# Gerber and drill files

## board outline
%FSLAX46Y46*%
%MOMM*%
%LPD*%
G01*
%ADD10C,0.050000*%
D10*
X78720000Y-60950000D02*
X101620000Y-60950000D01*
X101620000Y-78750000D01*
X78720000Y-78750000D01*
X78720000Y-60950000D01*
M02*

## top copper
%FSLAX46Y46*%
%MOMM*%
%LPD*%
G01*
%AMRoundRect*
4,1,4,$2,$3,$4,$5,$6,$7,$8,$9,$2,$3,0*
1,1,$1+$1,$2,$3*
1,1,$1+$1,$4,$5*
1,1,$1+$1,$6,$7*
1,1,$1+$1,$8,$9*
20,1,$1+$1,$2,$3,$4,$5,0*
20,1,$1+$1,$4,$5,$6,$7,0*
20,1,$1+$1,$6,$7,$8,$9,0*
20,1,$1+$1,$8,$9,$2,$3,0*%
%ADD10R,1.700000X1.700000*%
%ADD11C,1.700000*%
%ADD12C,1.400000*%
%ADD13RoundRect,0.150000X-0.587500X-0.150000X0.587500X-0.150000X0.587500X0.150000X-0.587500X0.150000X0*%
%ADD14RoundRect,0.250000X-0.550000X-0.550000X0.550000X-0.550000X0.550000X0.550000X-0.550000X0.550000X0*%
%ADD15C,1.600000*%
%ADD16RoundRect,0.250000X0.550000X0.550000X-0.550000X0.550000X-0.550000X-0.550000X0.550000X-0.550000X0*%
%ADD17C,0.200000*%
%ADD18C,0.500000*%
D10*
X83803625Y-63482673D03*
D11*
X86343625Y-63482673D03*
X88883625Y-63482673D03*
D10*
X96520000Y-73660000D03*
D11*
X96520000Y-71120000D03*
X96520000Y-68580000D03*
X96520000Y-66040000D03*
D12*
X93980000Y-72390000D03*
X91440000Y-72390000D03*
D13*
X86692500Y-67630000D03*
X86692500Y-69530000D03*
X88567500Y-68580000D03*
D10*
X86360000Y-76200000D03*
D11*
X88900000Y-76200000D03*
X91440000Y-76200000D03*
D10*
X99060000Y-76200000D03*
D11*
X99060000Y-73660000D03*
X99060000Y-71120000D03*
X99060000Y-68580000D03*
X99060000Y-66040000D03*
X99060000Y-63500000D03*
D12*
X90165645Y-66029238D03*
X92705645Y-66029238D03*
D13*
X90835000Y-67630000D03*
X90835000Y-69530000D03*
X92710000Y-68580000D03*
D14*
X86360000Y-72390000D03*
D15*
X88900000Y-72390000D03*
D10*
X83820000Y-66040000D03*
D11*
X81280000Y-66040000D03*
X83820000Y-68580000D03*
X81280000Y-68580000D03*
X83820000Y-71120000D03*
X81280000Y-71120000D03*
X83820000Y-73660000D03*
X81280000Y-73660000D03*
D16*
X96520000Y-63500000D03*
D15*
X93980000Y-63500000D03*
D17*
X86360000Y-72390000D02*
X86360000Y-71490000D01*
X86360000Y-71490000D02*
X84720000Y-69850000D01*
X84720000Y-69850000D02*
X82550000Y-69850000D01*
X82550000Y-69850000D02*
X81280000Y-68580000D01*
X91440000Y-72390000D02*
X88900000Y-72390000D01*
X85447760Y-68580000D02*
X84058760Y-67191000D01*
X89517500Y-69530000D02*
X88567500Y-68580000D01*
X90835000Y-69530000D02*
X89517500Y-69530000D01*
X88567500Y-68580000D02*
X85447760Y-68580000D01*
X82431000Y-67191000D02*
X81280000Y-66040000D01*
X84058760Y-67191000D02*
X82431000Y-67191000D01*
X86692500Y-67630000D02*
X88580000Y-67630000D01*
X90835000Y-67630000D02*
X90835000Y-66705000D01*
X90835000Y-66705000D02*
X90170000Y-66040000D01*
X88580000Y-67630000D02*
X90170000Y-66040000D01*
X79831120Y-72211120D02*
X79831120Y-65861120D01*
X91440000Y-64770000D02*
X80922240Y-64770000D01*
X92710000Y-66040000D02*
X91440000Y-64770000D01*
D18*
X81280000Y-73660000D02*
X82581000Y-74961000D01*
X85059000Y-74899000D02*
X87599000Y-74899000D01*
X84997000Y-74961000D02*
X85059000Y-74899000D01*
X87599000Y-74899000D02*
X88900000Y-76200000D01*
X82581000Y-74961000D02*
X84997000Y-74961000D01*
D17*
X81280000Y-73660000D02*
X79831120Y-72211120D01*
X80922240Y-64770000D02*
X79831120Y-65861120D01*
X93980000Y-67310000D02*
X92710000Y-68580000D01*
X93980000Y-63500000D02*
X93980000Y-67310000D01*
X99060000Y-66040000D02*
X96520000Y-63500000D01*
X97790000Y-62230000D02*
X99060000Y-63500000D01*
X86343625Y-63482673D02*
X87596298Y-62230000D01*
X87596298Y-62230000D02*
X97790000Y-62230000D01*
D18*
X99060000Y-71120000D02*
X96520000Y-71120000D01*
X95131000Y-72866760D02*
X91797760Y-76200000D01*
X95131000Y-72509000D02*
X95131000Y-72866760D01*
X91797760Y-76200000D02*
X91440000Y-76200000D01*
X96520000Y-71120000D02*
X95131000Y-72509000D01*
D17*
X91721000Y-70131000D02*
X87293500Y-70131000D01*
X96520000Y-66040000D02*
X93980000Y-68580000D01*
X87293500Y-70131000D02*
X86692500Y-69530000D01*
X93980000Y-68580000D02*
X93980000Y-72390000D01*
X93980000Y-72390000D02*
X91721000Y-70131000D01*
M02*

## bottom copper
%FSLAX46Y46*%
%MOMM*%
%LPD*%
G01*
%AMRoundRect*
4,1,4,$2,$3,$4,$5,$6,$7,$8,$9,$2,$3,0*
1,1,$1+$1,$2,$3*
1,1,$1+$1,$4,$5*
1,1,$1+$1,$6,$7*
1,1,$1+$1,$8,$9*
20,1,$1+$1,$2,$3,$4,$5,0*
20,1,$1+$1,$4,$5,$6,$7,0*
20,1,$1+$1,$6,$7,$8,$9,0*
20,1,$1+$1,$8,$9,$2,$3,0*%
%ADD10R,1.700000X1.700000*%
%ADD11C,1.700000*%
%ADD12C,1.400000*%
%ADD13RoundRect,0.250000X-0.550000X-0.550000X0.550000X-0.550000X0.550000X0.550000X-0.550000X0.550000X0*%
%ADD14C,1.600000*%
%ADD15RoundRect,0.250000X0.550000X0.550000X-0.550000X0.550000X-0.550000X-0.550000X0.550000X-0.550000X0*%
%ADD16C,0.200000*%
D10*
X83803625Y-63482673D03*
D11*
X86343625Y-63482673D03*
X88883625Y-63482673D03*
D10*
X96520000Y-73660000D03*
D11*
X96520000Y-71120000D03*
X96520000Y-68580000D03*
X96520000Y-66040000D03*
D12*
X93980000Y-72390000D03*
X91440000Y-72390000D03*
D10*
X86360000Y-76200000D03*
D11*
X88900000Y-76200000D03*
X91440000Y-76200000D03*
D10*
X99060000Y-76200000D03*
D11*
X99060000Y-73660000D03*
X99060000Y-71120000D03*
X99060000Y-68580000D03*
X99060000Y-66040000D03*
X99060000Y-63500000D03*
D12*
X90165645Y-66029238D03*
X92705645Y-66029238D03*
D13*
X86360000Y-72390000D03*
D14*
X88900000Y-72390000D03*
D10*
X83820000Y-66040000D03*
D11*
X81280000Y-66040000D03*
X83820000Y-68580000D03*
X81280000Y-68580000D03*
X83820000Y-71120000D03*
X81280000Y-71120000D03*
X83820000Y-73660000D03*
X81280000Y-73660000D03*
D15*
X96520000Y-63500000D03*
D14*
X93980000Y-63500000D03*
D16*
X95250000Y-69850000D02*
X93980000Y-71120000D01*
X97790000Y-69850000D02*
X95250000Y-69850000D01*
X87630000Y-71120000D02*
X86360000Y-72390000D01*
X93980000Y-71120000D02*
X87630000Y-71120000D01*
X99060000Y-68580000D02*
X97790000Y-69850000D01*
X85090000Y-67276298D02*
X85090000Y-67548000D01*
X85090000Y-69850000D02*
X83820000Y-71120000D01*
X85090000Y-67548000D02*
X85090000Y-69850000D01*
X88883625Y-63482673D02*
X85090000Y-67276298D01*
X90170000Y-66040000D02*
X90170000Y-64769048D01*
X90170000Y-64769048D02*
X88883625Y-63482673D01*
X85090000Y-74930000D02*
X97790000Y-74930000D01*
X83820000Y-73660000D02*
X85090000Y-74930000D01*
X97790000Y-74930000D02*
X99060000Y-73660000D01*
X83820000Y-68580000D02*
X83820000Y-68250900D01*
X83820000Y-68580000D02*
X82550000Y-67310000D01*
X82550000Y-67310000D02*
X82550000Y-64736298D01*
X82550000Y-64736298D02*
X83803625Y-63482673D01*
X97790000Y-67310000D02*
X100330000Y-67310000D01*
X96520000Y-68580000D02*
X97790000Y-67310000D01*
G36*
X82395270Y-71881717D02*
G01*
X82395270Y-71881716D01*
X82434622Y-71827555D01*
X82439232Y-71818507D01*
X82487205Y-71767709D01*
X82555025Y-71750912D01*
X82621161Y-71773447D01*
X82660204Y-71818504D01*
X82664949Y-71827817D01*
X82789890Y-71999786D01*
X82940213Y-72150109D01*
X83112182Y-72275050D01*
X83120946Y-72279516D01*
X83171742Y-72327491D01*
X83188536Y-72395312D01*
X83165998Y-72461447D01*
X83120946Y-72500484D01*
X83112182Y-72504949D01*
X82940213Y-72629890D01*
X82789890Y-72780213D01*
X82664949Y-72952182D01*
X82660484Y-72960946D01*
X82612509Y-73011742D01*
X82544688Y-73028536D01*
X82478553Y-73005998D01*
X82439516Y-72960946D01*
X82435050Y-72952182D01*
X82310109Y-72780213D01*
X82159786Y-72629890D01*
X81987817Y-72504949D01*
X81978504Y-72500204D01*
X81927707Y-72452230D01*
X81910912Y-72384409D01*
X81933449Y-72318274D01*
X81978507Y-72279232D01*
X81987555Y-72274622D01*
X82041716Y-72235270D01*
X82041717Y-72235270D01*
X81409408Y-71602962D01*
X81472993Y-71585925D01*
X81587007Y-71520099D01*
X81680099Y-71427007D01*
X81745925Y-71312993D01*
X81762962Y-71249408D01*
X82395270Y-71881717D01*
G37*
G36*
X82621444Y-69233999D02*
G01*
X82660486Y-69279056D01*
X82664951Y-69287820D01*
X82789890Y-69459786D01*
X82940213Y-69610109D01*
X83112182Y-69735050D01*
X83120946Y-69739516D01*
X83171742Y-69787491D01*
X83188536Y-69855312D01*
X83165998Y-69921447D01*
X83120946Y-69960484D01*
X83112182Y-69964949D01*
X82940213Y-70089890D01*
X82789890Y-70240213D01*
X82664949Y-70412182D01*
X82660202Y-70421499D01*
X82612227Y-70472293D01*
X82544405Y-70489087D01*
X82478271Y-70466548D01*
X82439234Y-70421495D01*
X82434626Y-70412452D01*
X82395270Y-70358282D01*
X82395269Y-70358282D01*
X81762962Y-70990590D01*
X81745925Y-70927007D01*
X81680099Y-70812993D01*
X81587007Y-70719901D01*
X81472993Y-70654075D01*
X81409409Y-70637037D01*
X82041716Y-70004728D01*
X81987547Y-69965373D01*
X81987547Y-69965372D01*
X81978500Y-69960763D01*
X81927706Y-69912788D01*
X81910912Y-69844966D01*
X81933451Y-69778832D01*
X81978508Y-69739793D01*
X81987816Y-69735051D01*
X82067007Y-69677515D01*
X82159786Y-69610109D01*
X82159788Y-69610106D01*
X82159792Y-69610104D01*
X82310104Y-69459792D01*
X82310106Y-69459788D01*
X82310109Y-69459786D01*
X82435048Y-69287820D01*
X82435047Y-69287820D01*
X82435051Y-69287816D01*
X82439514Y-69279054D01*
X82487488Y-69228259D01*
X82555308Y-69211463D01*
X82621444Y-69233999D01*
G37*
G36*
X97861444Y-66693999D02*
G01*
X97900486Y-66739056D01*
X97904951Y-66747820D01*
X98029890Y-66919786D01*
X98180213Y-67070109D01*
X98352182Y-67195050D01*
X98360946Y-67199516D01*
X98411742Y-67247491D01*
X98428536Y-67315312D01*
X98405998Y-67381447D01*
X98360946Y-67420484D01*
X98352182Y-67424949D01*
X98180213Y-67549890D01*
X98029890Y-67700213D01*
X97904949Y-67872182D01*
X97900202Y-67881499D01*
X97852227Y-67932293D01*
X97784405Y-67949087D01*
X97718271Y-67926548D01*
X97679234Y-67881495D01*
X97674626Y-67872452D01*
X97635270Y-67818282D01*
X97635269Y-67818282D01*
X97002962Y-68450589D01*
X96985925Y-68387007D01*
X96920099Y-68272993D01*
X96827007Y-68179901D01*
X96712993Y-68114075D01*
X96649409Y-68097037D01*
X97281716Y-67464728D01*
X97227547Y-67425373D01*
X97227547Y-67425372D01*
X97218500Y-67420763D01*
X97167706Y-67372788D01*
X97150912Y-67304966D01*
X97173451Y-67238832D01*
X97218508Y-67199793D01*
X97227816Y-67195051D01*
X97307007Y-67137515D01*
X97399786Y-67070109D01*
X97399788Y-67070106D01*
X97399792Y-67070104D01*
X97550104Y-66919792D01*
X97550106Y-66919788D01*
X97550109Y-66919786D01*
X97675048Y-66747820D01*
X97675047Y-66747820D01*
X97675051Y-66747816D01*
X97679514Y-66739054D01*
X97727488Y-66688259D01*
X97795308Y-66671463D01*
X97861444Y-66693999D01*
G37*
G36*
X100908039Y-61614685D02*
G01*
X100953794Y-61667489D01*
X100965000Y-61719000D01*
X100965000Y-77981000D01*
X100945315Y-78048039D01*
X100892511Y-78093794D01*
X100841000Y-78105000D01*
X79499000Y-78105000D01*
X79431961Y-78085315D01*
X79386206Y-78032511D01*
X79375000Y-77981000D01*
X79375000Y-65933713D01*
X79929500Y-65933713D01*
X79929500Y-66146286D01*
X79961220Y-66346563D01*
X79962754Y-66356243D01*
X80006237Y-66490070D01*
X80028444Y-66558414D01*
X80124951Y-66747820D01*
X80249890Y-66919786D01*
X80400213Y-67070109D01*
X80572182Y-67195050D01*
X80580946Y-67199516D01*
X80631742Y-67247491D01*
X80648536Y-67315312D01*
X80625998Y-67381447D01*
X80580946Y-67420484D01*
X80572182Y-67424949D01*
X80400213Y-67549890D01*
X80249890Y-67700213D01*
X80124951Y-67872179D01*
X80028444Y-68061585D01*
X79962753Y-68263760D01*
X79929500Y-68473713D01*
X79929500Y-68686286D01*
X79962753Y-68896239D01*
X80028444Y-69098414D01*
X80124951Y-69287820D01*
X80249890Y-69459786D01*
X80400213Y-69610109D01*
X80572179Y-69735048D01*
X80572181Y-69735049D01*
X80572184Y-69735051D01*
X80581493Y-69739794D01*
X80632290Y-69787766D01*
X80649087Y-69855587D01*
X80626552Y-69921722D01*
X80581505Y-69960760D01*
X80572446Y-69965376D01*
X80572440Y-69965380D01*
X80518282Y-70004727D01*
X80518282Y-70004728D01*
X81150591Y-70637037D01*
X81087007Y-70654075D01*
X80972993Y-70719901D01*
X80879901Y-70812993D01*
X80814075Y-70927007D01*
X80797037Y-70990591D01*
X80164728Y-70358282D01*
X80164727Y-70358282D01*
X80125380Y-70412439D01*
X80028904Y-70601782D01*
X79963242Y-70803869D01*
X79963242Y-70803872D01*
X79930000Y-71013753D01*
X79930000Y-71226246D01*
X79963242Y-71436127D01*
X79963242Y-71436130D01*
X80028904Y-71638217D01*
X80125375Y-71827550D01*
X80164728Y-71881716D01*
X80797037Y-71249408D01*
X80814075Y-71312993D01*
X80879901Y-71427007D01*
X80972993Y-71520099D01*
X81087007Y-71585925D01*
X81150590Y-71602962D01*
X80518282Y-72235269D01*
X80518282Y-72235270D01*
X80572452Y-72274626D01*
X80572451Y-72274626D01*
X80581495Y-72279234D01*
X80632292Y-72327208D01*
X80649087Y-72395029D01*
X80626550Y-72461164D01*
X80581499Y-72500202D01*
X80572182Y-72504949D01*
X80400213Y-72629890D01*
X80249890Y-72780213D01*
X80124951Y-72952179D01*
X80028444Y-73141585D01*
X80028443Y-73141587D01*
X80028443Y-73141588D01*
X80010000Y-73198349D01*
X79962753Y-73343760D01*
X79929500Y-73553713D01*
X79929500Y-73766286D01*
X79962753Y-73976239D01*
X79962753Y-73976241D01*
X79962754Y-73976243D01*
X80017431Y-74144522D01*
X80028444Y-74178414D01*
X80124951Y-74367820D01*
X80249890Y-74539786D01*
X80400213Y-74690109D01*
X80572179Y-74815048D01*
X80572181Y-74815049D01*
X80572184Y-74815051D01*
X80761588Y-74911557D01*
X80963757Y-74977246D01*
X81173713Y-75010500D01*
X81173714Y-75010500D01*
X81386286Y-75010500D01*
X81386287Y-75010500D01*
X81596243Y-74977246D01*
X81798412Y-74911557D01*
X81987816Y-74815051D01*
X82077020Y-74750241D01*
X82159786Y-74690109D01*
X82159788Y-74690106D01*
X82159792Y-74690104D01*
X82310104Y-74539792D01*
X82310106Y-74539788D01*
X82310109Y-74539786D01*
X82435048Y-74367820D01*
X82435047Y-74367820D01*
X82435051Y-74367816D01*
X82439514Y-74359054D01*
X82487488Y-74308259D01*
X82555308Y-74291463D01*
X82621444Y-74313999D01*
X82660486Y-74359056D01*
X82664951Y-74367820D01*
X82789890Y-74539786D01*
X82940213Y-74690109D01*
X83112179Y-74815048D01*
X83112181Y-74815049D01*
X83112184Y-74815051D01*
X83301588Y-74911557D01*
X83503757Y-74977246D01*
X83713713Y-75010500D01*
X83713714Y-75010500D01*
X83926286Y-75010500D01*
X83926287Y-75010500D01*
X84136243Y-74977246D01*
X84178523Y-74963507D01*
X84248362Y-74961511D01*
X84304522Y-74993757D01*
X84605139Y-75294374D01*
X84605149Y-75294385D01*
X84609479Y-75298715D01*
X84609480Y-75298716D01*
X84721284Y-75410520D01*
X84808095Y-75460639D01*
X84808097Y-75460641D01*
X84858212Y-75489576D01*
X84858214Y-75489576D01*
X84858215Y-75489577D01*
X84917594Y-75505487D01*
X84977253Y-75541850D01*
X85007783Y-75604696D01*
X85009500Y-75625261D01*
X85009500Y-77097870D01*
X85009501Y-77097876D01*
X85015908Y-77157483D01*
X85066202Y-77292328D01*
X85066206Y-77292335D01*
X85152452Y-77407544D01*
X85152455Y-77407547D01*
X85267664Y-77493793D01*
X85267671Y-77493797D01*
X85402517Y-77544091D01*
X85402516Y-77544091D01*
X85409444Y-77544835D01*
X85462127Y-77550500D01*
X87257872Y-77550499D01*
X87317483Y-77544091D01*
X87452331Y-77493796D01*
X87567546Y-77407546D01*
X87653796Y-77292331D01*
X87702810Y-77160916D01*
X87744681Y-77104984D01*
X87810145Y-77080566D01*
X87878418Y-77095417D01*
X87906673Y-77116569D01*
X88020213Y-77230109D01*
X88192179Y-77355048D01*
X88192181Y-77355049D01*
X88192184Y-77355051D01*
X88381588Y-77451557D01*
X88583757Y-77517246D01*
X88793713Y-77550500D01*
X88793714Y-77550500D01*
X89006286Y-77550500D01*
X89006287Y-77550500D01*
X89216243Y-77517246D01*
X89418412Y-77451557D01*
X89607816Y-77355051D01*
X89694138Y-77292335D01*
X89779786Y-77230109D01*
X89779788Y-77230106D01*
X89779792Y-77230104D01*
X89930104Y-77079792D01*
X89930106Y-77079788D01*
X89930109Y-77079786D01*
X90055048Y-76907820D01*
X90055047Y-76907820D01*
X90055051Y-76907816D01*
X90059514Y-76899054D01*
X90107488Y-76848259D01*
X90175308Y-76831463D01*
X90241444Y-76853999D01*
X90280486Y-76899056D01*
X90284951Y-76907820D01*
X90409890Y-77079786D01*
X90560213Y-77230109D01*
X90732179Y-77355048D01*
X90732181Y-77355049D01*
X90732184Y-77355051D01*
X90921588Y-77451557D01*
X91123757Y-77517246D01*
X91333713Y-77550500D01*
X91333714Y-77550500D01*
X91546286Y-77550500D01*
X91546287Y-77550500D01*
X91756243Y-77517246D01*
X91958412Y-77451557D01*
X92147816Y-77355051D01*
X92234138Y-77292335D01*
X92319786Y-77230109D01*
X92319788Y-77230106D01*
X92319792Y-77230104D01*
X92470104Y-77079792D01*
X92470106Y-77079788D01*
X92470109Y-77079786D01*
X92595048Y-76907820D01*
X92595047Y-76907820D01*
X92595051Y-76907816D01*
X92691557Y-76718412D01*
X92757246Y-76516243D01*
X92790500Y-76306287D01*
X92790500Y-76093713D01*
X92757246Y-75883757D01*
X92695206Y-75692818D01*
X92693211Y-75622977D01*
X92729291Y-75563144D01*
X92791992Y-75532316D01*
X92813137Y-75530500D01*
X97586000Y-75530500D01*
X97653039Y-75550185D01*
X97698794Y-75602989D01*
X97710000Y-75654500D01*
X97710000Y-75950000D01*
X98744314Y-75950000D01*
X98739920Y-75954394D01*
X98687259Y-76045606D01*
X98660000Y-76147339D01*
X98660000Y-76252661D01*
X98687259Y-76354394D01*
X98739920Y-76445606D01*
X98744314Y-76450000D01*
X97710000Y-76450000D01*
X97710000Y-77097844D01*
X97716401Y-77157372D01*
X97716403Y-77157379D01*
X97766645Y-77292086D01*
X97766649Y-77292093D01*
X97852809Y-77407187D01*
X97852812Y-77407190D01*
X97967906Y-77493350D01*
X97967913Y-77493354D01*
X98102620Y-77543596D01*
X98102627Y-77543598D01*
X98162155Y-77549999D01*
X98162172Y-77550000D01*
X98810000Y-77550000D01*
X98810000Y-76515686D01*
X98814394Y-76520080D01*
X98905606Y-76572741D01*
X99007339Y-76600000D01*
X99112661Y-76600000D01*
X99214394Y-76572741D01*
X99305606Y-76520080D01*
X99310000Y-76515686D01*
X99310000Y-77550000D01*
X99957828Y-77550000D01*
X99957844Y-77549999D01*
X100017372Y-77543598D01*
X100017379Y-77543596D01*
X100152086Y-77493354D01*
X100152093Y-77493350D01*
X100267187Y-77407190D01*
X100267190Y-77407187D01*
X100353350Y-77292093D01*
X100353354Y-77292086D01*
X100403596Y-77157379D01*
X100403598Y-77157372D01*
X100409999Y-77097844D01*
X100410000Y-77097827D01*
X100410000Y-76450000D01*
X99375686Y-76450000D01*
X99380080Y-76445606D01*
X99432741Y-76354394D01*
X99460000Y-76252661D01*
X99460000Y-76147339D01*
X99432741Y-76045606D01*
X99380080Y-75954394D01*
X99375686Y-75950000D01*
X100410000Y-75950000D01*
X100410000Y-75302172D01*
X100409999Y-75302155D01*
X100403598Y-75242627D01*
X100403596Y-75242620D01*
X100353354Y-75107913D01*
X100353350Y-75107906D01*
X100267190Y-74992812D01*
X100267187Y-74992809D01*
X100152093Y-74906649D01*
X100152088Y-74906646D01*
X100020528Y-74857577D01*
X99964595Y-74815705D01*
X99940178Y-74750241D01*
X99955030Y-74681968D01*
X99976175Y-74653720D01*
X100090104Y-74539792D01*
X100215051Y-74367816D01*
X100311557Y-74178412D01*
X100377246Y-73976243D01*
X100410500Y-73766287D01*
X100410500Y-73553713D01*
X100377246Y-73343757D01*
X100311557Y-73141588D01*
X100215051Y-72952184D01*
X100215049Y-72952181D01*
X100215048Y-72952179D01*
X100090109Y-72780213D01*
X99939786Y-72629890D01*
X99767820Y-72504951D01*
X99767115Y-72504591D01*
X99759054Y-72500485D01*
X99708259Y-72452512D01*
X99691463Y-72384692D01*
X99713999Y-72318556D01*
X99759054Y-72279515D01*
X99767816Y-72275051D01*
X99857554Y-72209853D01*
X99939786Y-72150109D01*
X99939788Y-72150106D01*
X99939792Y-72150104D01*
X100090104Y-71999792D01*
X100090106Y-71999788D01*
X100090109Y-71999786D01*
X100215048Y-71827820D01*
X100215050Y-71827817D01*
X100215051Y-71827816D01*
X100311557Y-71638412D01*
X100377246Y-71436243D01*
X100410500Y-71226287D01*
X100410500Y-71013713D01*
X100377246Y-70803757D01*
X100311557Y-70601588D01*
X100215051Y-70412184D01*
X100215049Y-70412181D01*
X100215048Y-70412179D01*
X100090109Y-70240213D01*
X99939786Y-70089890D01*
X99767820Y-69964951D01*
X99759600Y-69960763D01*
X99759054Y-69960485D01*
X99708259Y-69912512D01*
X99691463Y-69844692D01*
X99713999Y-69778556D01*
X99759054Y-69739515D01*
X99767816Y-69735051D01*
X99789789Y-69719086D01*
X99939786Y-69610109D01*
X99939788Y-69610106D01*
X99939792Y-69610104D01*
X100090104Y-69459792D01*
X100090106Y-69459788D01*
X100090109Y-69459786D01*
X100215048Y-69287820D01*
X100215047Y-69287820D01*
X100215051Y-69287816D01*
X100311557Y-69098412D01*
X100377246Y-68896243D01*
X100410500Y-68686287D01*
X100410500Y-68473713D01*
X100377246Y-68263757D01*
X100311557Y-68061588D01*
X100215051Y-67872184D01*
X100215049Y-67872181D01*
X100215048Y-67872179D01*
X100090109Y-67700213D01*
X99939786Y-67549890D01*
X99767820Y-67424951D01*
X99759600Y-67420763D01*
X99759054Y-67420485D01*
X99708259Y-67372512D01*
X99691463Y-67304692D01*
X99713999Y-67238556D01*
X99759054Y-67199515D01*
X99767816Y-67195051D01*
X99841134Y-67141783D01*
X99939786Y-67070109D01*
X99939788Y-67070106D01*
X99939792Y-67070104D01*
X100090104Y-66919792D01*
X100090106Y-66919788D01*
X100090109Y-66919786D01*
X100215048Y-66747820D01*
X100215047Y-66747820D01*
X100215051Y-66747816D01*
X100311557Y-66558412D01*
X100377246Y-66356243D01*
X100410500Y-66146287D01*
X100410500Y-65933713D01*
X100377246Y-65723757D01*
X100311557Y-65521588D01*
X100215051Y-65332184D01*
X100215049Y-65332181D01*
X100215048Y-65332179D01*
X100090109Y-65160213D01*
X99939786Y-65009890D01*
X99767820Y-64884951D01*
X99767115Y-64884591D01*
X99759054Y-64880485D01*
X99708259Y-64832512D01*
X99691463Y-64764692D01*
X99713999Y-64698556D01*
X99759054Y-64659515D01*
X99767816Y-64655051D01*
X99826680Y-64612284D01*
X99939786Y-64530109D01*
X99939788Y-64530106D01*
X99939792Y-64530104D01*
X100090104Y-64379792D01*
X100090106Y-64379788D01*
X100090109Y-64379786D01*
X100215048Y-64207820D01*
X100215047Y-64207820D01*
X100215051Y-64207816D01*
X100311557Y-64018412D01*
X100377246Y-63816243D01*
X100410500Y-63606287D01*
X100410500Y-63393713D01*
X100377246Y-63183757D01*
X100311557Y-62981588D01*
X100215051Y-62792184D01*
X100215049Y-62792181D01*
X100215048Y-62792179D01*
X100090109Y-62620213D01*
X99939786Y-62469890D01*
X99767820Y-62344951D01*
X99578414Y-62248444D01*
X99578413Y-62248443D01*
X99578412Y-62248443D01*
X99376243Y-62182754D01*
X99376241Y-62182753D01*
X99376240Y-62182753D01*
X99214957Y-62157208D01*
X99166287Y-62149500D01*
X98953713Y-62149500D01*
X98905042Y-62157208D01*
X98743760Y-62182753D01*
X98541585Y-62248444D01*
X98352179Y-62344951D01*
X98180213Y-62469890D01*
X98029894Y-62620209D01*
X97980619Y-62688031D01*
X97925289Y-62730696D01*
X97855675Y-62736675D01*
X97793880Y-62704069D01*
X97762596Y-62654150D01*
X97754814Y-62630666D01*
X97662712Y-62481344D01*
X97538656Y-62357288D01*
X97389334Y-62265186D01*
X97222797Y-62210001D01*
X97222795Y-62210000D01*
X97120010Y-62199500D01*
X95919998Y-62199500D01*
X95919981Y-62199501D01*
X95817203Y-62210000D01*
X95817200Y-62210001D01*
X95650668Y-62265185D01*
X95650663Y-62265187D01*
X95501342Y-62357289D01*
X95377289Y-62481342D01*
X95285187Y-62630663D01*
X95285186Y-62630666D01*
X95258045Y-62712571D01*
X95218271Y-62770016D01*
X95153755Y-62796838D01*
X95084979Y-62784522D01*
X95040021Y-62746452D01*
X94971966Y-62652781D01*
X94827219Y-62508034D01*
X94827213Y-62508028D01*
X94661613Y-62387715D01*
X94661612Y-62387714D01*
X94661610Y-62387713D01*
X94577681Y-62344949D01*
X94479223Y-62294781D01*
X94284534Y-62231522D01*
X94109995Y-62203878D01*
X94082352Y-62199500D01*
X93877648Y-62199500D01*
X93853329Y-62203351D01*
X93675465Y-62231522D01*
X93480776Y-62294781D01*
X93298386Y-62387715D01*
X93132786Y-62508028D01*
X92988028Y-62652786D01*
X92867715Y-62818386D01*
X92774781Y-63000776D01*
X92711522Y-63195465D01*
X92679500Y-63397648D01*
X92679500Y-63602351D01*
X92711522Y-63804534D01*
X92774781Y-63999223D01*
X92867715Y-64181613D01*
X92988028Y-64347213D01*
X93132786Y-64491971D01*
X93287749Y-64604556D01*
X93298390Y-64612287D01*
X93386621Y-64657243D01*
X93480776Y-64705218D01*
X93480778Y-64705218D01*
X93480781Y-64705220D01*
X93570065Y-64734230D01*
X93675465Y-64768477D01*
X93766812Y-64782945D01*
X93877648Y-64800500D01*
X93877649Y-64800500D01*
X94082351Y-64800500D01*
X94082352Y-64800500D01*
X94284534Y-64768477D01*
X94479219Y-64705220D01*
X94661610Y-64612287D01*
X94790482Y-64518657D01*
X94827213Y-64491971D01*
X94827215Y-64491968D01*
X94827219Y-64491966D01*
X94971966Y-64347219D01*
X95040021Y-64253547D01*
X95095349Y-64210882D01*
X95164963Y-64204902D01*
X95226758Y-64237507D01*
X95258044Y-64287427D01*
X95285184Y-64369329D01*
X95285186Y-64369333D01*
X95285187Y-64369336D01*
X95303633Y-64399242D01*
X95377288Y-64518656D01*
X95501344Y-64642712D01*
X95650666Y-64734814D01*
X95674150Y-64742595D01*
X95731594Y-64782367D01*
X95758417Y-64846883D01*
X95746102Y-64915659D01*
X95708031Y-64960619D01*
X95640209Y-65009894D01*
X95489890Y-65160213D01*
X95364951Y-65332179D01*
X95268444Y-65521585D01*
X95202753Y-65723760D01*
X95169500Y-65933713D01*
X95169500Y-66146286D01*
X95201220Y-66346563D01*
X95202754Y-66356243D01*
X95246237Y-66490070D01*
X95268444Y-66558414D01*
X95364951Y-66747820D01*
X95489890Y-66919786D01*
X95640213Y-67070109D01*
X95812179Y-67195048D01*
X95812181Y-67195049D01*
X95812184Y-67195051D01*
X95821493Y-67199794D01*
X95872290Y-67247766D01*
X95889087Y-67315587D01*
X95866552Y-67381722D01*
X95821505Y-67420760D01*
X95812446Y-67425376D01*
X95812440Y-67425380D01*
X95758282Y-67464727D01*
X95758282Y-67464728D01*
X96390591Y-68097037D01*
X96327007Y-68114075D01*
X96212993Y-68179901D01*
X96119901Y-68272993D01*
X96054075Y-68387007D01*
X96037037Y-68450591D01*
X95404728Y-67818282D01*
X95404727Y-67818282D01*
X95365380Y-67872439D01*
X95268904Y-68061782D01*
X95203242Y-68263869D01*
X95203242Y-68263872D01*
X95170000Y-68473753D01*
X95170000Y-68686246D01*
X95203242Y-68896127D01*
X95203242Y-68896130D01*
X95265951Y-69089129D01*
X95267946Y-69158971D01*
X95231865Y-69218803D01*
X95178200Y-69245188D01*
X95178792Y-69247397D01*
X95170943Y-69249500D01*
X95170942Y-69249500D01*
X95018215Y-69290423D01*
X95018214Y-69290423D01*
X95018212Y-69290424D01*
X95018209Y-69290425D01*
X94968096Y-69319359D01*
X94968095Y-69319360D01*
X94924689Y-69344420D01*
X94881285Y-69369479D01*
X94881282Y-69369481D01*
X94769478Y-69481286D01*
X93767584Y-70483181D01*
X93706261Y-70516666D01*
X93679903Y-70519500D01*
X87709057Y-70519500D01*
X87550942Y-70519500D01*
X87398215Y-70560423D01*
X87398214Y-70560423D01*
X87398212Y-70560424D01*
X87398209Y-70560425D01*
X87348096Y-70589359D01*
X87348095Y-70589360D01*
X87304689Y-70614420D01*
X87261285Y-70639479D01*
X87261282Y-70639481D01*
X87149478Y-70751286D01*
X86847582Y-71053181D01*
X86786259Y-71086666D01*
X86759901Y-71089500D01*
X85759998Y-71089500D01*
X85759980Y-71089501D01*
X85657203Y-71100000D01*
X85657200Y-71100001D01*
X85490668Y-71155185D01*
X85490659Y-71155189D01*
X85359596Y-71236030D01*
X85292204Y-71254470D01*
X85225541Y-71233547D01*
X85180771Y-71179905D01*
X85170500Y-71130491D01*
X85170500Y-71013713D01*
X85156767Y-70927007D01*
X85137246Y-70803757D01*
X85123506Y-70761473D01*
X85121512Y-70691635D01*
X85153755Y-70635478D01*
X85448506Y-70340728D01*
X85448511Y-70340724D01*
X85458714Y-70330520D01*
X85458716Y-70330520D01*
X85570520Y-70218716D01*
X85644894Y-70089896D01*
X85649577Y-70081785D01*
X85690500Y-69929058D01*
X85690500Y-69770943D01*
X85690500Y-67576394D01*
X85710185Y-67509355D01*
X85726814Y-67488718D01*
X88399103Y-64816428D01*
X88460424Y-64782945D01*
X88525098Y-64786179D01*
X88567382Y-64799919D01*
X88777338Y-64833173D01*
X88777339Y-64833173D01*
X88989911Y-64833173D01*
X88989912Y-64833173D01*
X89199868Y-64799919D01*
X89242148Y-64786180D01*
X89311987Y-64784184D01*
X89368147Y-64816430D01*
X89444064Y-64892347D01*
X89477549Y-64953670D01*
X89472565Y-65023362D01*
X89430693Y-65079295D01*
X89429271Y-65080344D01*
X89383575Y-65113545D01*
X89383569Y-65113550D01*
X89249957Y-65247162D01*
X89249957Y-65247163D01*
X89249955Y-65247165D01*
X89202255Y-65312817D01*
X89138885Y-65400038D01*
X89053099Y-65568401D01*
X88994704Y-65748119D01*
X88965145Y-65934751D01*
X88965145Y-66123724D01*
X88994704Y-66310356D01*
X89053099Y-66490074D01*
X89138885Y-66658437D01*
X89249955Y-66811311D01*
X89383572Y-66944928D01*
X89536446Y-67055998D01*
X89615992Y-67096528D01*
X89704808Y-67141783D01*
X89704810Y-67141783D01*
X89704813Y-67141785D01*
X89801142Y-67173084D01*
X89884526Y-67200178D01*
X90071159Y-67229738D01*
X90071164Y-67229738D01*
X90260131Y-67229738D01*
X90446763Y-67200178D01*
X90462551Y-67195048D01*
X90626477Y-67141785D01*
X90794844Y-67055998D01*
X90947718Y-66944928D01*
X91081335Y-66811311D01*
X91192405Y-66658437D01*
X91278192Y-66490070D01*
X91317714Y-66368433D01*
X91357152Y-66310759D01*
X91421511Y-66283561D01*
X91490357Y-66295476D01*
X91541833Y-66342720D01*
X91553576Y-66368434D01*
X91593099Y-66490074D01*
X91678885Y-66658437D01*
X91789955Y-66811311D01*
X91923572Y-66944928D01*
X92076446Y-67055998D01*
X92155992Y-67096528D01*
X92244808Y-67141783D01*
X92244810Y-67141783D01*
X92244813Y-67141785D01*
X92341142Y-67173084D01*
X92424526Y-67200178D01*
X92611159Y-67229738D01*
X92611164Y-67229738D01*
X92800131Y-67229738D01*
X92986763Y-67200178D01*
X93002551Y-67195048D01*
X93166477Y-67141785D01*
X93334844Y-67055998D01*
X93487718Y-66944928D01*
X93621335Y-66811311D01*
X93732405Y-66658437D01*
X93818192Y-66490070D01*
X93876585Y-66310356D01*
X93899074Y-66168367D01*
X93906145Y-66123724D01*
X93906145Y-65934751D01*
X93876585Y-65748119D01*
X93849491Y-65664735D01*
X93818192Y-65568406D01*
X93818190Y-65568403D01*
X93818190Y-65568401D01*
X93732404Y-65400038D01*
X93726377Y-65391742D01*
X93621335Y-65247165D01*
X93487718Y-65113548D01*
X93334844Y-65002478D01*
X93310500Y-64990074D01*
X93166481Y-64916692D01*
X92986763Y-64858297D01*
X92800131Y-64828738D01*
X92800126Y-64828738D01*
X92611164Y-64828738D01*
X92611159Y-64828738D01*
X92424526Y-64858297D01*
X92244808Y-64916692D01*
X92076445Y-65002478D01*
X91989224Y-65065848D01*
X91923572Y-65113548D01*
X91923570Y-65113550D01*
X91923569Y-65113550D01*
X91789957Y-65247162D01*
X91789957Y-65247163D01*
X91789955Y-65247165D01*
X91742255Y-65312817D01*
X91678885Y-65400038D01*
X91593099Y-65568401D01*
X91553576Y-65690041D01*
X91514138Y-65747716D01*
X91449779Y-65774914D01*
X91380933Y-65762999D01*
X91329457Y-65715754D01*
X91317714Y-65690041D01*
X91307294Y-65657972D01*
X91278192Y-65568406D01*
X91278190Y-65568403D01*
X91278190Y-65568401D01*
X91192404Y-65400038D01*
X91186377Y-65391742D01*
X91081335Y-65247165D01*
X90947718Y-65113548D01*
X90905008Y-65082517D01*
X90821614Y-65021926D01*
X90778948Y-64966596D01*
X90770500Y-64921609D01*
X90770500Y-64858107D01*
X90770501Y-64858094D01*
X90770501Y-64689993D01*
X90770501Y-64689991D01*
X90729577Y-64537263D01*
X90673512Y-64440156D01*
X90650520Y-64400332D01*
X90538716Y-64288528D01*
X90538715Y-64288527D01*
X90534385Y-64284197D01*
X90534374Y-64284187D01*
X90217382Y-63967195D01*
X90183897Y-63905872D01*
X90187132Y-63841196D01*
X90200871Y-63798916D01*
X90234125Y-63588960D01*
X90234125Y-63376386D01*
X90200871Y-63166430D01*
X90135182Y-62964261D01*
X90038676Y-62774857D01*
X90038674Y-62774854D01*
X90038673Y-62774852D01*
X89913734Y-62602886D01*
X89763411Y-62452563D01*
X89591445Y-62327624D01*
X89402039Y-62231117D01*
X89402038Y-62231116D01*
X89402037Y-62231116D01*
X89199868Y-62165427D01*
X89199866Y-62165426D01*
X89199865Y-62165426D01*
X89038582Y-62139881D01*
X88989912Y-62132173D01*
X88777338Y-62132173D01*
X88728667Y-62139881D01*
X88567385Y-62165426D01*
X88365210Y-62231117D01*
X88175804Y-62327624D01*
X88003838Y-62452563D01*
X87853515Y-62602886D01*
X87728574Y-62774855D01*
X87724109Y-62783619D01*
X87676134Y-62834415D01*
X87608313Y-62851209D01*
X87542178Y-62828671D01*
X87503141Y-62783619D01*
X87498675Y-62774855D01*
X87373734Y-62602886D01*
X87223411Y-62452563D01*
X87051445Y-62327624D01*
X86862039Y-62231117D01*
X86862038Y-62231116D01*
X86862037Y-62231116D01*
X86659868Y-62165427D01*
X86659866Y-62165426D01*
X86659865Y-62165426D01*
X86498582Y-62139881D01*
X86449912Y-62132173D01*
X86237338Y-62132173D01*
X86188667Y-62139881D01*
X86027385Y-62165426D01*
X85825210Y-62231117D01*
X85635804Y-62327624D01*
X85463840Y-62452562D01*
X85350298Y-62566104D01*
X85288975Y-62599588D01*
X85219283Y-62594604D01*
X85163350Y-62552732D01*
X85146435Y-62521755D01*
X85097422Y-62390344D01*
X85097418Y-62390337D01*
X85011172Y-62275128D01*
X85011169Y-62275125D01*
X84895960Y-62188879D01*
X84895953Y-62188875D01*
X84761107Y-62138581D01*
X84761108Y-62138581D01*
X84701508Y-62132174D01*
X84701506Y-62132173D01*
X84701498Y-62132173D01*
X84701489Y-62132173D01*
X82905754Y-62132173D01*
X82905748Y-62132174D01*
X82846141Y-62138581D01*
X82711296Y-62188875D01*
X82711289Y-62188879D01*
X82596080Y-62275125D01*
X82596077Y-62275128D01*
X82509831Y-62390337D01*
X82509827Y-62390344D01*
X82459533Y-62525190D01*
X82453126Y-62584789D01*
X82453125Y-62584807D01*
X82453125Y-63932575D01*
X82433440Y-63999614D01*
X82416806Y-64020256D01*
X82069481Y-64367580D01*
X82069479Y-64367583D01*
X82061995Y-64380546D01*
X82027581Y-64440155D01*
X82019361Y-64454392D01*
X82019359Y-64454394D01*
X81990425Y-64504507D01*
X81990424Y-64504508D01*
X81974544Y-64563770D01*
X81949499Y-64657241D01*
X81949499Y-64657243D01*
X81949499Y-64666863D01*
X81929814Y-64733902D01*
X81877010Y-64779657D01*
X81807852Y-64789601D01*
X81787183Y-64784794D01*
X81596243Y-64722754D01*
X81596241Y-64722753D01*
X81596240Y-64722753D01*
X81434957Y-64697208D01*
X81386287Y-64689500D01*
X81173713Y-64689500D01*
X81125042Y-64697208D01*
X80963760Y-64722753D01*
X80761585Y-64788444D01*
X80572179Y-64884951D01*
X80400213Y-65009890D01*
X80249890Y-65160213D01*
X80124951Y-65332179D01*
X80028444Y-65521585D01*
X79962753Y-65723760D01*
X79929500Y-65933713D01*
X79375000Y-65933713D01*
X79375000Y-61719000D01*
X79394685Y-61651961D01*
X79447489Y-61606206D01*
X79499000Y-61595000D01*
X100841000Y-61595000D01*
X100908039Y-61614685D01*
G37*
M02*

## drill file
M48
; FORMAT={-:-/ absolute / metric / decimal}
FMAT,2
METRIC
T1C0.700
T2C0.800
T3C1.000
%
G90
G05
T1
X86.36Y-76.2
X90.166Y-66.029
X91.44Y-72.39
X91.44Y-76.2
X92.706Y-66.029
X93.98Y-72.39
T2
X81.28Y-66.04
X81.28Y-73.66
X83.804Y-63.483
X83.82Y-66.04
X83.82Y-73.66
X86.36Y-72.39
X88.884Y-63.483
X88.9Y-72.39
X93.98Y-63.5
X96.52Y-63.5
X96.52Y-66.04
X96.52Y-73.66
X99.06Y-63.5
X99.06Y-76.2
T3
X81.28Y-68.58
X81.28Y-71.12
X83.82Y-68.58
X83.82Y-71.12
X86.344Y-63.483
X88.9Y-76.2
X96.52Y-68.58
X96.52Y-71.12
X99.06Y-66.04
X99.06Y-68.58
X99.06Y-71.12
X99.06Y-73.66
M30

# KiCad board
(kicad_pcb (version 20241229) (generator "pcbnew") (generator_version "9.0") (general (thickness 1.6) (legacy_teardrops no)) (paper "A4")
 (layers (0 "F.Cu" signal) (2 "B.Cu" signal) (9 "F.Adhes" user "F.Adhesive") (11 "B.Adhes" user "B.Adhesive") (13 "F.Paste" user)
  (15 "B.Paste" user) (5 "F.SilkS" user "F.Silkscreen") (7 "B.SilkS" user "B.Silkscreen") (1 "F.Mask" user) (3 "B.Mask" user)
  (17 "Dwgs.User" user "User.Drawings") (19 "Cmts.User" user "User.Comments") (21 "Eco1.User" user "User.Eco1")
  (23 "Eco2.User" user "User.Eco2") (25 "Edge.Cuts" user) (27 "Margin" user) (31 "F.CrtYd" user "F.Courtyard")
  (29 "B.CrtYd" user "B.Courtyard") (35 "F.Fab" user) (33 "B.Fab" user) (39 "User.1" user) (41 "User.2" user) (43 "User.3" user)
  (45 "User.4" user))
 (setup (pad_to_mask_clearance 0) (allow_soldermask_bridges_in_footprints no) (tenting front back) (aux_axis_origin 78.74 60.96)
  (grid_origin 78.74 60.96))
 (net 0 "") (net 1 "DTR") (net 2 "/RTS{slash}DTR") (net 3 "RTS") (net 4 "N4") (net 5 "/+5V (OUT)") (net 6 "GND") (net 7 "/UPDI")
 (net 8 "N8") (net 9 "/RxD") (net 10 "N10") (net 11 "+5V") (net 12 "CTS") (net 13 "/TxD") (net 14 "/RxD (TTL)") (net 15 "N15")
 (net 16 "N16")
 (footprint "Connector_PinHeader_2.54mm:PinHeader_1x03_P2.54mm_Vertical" (layer "F.Cu") (at 83.803625 63.482673 90)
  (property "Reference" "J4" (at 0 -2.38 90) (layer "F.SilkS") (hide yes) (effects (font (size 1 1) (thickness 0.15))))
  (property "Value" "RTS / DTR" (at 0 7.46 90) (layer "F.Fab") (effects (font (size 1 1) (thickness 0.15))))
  (pad "1" thru_hole rect (at 0 0 90) (size 1.7 1.7) (drill 0.8) (layers "*.Cu" "*.Mask") (remove_unused_layers no) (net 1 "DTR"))
  (pad "2" thru_hole circle (at 0 2.54 90) (size 1.7 1.7) (drill 1) (layers "*.Cu" "*.Mask") (remove_unused_layers no)
   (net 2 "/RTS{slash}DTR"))
  (pad "3" thru_hole circle (at 0 5.08 90) (size 1.7 1.7) (drill 0.8) (layers "*.Cu" "*.Mask") (remove_unused_layers no) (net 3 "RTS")))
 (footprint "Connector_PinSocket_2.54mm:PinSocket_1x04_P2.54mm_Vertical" (layer "F.Cu") (at 96.52 73.66 180)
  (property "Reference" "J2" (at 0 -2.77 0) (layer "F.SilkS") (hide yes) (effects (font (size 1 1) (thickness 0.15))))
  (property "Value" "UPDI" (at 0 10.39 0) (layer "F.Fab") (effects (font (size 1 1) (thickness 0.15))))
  (pad "1" thru_hole rect (at 0 0 180) (size 1.7 1.7) (drill 0.8) (layers "*.Cu" "*.Mask") (remove_unused_layers no) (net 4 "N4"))
  (pad "2" thru_hole circle (at 0 2.54 180) (size 1.7 1.7) (drill 1) (layers "*.Cu" "*.Mask") (remove_unused_layers no) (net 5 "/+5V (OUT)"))
  (pad "3" thru_hole circle (at 0 5.08 180) (size 1.7 1.7) (drill 1) (layers "*.Cu" "*.Mask") (remove_unused_layers no) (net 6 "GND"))
  (pad "4" thru_hole circle (at 0 7.62 180) (size 1.7 1.7) (drill 0.8) (layers "*.Cu" "*.Mask") (remove_unused_layers no) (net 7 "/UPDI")))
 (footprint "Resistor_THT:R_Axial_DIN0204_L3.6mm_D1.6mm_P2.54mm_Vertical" (layer "F.Cu") (at 93.98 72.39 180)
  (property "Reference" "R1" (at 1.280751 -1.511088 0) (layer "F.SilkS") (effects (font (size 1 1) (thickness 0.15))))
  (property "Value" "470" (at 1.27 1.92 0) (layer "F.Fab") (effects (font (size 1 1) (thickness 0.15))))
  (pad "1" thru_hole circle (at 0 0 180) (size 1.4 1.4) (drill 0.7) (layers "*.Cu" "*.Mask") (remove_unused_layers no) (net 7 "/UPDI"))
  (pad "2" thru_hole circle (at 2.54 0 180) (size 1.4 1.4) (drill 0.7) (layers "*.Cu" "*.Mask") (remove_unused_layers no) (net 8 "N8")))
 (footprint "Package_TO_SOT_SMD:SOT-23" (layer "F.Cu") (at 87.63 68.58)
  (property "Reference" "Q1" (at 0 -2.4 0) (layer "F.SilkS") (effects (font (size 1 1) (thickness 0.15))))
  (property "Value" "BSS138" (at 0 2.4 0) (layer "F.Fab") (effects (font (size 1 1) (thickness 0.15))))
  (pad "1" smd roundrect (at -0.9375 -0.95) (size 1.475 0.6) (layers "F.Cu" "F.Mask" "F.Paste") (roundrect_rratio 0.25) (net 3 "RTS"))
  (pad "2" smd roundrect (at -0.9375 0.95) (size 1.475 0.6) (layers "F.Cu" "F.Mask" "F.Paste") (roundrect_rratio 0.25) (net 7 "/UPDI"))
  (pad "3" smd roundrect (at 0.9375 0) (size 1.475 0.6) (layers "F.Cu" "F.Mask" "F.Paste") (roundrect_rratio 0.25) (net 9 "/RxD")))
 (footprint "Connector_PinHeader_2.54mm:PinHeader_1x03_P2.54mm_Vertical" (layer "F.Cu") (at 86.36 76.2 90)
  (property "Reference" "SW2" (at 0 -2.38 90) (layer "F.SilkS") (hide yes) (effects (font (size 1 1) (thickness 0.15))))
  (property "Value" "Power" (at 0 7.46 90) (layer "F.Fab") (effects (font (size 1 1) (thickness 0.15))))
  (pad "1" thru_hole rect (at 0 0 90) (size 1.7 1.7) (drill 0.7) (layers "*.Cu" "*.Mask") (remove_unused_layers no) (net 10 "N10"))
  (pad "2" thru_hole circle (at 0 2.54 90) (size 1.7 1.7) (drill 1) (layers "*.Cu" "*.Mask") (remove_unused_layers no) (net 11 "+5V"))
  (pad "3" thru_hole circle (at 0 5.08 90) (size 1.7 1.7) (drill 0.7) (layers "*.Cu" "*.Mask") (remove_unused_layers no)
   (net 5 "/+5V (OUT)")))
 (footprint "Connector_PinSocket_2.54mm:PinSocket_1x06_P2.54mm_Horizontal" (layer "F.Cu") (at 99.06 76.2 180)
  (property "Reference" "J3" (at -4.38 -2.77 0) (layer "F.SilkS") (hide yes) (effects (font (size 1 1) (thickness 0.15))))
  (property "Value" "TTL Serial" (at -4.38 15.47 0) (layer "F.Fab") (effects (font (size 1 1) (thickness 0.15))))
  (pad "1" thru_hole rect (at 0 0 180) (size 1.7 1.7) (drill 0.8) (layers "*.Cu" "*.Mask") (remove_unused_layers no) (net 6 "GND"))
  (pad "2" thru_hole circle (at 0 2.54 180) (size 1.7 1.7) (drill 1) (layers "*.Cu" "*.Mask") (remove_unused_layers no) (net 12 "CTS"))
  (pad "3" thru_hole circle (at 0 5.08 180) (size 1.7 1.7) (drill 1) (layers "*.Cu" "*.Mask") (remove_unused_layers no) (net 5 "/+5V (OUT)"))
  (pad "4" thru_hole circle (at 0 7.62 180) (size 1.7 1.7) (drill 1) (layers "*.Cu" "*.Mask") (remove_unused_layers no) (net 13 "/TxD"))
  (pad "5" thru_hole circle (at 0 10.16 180) (size 1.7 1.7) (drill 1) (layers "*.Cu" "*.Mask") (remove_unused_layers no)
   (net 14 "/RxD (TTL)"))
  (pad "6" thru_hole circle (at 0 12.7 180) (size 1.7 1.7) (drill 0.8) (layers "*.Cu" "*.Mask") (remove_unused_layers no)
   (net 2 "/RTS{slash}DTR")))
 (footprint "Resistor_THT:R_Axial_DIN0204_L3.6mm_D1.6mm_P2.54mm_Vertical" (layer "F.Cu") (at 90.165645 66.029238)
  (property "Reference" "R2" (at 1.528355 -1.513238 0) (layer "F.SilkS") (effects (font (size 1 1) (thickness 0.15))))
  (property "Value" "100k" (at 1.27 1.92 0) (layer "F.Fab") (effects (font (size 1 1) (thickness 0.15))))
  (pad "1" thru_hole circle (at 0 0) (size 1.4 1.4) (drill 0.7) (layers "*.Cu" "*.Mask") (remove_unused_layers no) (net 3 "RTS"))
  (pad "2" thru_hole circle (at 2.54 0) (size 1.4 1.4) (drill 0.7) (layers "*.Cu" "*.Mask") (remove_unused_layers no) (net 11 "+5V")))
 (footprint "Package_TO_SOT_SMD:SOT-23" (layer "F.Cu") (at 91.7725 68.58)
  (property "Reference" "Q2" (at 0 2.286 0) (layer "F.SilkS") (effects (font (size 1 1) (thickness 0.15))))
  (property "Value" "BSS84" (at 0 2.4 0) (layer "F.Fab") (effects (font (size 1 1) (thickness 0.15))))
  (pad "1" smd roundrect (at -0.9375 -0.95) (size 1.475 0.6) (layers "F.Cu" "F.Mask" "F.Paste") (roundrect_rratio 0.25) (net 3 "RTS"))
  (pad "2" smd roundrect (at -0.9375 0.95) (size 1.475 0.6) (layers "F.Cu" "F.Mask" "F.Paste") (roundrect_rratio 0.25) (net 9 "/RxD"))
  (pad "3" smd roundrect (at 0.9375 0) (size 1.475 0.6) (layers "F.Cu" "F.Mask" "F.Paste") (roundrect_rratio 0.25) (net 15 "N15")))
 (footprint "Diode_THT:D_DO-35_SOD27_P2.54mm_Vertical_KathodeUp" (layer "F.Cu") (at 86.36 72.39)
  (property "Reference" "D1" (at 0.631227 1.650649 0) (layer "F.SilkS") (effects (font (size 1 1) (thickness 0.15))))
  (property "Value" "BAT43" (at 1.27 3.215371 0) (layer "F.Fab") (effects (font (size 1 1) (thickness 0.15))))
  (pad "1" thru_hole roundrect (at 0 0) (size 1.6 1.6) (drill 0.8) (layers "*.Cu" "*.Mask") (remove_unused_layers no)
   (roundrect_rratio 0.15625) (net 13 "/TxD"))
  (pad "2" thru_hole circle (at 2.54 0) (size 1.6 1.6) (drill 0.8) (layers "*.Cu" "*.Mask") (remove_unused_layers no) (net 8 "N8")))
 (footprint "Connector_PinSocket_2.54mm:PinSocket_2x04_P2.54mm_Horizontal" (layer "F.Cu") (at 83.82 66.04)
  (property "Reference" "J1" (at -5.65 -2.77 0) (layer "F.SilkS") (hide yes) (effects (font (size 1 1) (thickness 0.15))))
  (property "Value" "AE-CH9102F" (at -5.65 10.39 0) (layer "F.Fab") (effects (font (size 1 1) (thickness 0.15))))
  (pad "1" thru_hole rect (at 0 0) (size 1.7 1.7) (drill 0.8) (layers "*.Cu" "*.Mask") (remove_unused_layers no) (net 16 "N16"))
  (pad "2" thru_hole circle (at -2.54 0) (size 1.7 1.7) (drill 0.8) (layers "*.Cu" "*.Mask") (remove_unused_layers no) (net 9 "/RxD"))
  (pad "3" thru_hole circle (at 0 2.54) (size 1.7 1.7) (drill 1) (layers "*.Cu" "*.Mask") (remove_unused_layers no) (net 1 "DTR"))
  (pad "4" thru_hole circle (at -2.54 2.54) (size 1.7 1.7) (drill 1) (layers "*.Cu" "*.Mask") (remove_unused_layers no) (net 13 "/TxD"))
  (pad "5" thru_hole circle (at 0 5.08) (size 1.7 1.7) (drill 1) (layers "*.Cu" "*.Mask") (remove_unused_layers no) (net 3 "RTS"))
  (pad "6" thru_hole circle (at -2.54 5.08) (size 1.7 1.7) (drill 1) (layers "*.Cu" "*.Mask") (remove_unused_layers no) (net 6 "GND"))
  (pad "7" thru_hole circle (at 0 7.62) (size 1.7 1.7) (drill 0.8) (layers "*.Cu" "*.Mask") (remove_unused_layers no) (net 12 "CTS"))
  (pad "8" thru_hole circle (at -2.54 7.62) (size 1.7 1.7) (drill 0.8) (layers "*.Cu" "*.Mask") (remove_unused_layers no) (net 11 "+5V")))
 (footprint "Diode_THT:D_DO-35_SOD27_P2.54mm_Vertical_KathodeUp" (layer "F.Cu") (at 96.52 63.5 180)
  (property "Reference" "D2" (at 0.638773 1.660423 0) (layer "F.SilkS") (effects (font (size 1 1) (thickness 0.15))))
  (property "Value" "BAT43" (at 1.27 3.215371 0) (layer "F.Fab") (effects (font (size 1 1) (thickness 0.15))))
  (pad "1" thru_hole roundrect (at 0 0 180) (size 1.6 1.6) (drill 0.8) (layers "*.Cu" "*.Mask") (remove_unused_layers no)
   (roundrect_rratio 0.15625) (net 14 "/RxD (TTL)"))
  (pad "2" thru_hole circle (at 2.54 0 180) (size 1.6 1.6) (drill 0.8) (layers "*.Cu" "*.Mask") (remove_unused_layers no) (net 15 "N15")))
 (gr_rect (start 78.72 60.95) (end 101.62 78.75) (stroke (width 0.05) (type solid)) (fill no) (layer "Edge.Cuts"))
 (segment (start 86.36 72.39) (end 86.36 71.49) (width 0.2) (layer "F.Cu") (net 13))
 (segment (start 86.36 71.49) (end 84.72 69.85) (width 0.2) (layer "F.Cu") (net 13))
 (segment (start 84.72 69.85) (end 82.55 69.85) (width 0.2) (layer "F.Cu") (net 13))
 (segment (start 82.55 69.85) (end 81.28 68.58) (width 0.2) (layer "F.Cu") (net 13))
 (segment (start 95.25 69.85) (end 93.98 71.12) (width 0.2) (layer "B.Cu") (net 13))
 (segment (start 97.79 69.85) (end 95.25 69.85) (width 0.2) (layer "B.Cu") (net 13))
 (segment (start 87.63 71.12) (end 86.36 72.39) (width 0.2) (layer "B.Cu") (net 13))
 (segment (start 93.98 71.12) (end 87.63 71.12) (width 0.2) (layer "B.Cu") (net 13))
 (segment (start 99.06 68.58) (end 97.79 69.85) (width 0.2) (layer "B.Cu") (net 13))
 (segment (start 91.44 72.39) (end 88.9 72.39) (width 0.2) (layer "F.Cu") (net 8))
 (segment (start 85.44776 68.58) (end 84.05876 67.191) (width 0.2) (layer "F.Cu") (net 9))
 (segment (start 89.5175 69.53) (end 88.5675 68.58) (width 0.2) (layer "F.Cu") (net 9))
 (segment (start 90.835 69.53) (end 89.5175 69.53) (width 0.2) (layer "F.Cu") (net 9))
 (segment (start 88.5675 68.58) (end 85.44776 68.58) (width 0.2) (layer "F.Cu") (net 9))
 (segment (start 82.431 67.191) (end 81.28 66.04) (width 0.2) (layer "F.Cu") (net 9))
 (segment (start 84.05876 67.191) (end 82.431 67.191) (width 0.2) (layer "F.Cu") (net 9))
 (segment (start 86.6925 67.63) (end 88.58 67.63) (width 0.2) (layer "F.Cu") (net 3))
 (segment (start 90.835 67.63) (end 90.835 66.705) (width 0.2) (layer "F.Cu") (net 3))
 (segment (start 90.835 66.705) (end 90.17 66.04) (width 0.2) (layer "F.Cu") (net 3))
 (segment (start 88.58 67.63) (end 90.17 66.04) (width 0.2) (layer "F.Cu") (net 3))
 (segment (start 85.09 67.276298) (end 85.09 67.548) (width 0.2) (layer "B.Cu") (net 3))
 (segment (start 85.09 69.85) (end 83.82 71.12) (width 0.2) (layer "B.Cu") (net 3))
 (segment (start 85.09 67.548) (end 85.09 69.85) (width 0.2) (layer "B.Cu") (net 3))
 (segment (start 88.883625 63.482673) (end 85.09 67.276298) (width 0.2) (layer "B.Cu") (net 3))
 (segment (start 90.17 66.04) (end 90.17 64.769048) (width 0.2) (layer "B.Cu") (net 3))
 (segment (start 90.17 64.769048) (end 88.883625 63.482673) (width 0.2) (layer "B.Cu") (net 3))
 (segment (start 85.09 74.93) (end 97.79 74.93) (width 0.2) (layer "B.Cu") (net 12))
 (segment (start 83.82 73.66) (end 85.09 74.93) (width 0.2) (layer "B.Cu") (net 12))
 (segment (start 97.79 74.93) (end 99.06 73.66) (width 0.2) (layer "B.Cu") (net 12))
 (segment (start 83.82 68.58) (end 83.82 68.2509) (width 0.2) (layer "B.Cu") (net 1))
 (segment (start 83.82 68.58) (end 82.55 67.31) (width 0.2) (layer "B.Cu") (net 1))
 (segment (start 82.55 67.31) (end 82.55 64.736298) (width 0.2) (layer "B.Cu") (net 1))
 (segment (start 82.55 64.736298) (end 83.803625 63.482673) (width 0.2) (layer "B.Cu") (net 1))
 (segment (start 97.79 67.31) (end 100.33 67.31) (width 0.2) (layer "B.Cu") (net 6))
 (segment (start 96.52 68.58) (end 97.79 67.31) (width 0.2) (layer "B.Cu") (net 6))
 (segment (start 79.83112 72.21112) (end 79.83112 65.86112) (width 0.2) (layer "F.Cu") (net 11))
 (segment (start 91.44 64.77) (end 80.92224 64.77) (width 0.2) (layer "F.Cu") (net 11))
 (segment (start 92.71 66.04) (end 91.44 64.77) (width 0.2) (layer "F.Cu") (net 11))
 (segment (start 81.28 73.66) (end 82.581 74.961) (width 0.5) (layer "F.Cu") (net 11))
 (segment (start 85.059 74.899) (end 87.599 74.899) (width 0.5) (layer "F.Cu") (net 11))
 (segment (start 84.997 74.961) (end 85.059 74.899) (width 0.5) (layer "F.Cu") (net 11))
 (segment (start 87.599 74.899) (end 88.9 76.2) (width 0.5) (layer "F.Cu") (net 11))
 (segment (start 82.581 74.961) (end 84.997 74.961) (width 0.5) (layer "F.Cu") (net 11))
 (segment (start 81.28 73.66) (end 79.83112 72.21112) (width 0.2) (layer "F.Cu") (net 11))
 (segment (start 80.92224 64.77) (end 79.83112 65.86112) (width 0.2) (layer "F.Cu") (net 11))
 (segment (start 93.98 67.31) (end 92.71 68.58) (width 0.2) (layer "F.Cu") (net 15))
 (segment (start 93.98 63.5) (end 93.98 67.31) (width 0.2) (layer "F.Cu") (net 15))
 (segment (start 99.06 66.04) (end 96.52 63.5) (width 0.2) (layer "F.Cu") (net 14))
 (segment (start 97.79 62.23) (end 99.06 63.5) (width 0.2) (layer "F.Cu") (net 2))
 (segment (start 86.343625 63.482673) (end 87.596298 62.23) (width 0.2) (layer "F.Cu") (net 2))
 (segment (start 87.596298 62.23) (end 97.79 62.23) (width 0.2) (layer "F.Cu") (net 2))
 (segment (start 99.06 71.12) (end 96.52 71.12) (width 0.5) (layer "F.Cu") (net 5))
 (segment (start 95.131 72.86676) (end 91.79776 76.2) (width 0.5) (layer "F.Cu") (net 5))
 (segment (start 95.131 72.509) (end 95.131 72.86676) (width 0.5) (layer "F.Cu") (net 5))
 (segment (start 91.79776 76.2) (end 91.44 76.2) (width 0.5) (layer "F.Cu") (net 5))
 (segment (start 96.52 71.12) (end 95.131 72.509) (width 0.5) (layer "F.Cu") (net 5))
 (segment (start 91.721 70.131) (end 87.2935 70.131) (width 0.2) (layer "F.Cu") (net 7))
 (segment (start 96.52 66.04) (end 93.98 68.58) (width 0.2) (layer "F.Cu") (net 7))
 (segment (start 87.2935 70.131) (end 86.6925 69.53) (width 0.2) (layer "F.Cu") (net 7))
 (segment (start 93.98 68.58) (end 93.98 72.39) (width 0.2) (layer "F.Cu") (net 7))
 (segment (start 93.98 72.39) (end 91.721 70.131) (width 0.2) (layer "F.Cu") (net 7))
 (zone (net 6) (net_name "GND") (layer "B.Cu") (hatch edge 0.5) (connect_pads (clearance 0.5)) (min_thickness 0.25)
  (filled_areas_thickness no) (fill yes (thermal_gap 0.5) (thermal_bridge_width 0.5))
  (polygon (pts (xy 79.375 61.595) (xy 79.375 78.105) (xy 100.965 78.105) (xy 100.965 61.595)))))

